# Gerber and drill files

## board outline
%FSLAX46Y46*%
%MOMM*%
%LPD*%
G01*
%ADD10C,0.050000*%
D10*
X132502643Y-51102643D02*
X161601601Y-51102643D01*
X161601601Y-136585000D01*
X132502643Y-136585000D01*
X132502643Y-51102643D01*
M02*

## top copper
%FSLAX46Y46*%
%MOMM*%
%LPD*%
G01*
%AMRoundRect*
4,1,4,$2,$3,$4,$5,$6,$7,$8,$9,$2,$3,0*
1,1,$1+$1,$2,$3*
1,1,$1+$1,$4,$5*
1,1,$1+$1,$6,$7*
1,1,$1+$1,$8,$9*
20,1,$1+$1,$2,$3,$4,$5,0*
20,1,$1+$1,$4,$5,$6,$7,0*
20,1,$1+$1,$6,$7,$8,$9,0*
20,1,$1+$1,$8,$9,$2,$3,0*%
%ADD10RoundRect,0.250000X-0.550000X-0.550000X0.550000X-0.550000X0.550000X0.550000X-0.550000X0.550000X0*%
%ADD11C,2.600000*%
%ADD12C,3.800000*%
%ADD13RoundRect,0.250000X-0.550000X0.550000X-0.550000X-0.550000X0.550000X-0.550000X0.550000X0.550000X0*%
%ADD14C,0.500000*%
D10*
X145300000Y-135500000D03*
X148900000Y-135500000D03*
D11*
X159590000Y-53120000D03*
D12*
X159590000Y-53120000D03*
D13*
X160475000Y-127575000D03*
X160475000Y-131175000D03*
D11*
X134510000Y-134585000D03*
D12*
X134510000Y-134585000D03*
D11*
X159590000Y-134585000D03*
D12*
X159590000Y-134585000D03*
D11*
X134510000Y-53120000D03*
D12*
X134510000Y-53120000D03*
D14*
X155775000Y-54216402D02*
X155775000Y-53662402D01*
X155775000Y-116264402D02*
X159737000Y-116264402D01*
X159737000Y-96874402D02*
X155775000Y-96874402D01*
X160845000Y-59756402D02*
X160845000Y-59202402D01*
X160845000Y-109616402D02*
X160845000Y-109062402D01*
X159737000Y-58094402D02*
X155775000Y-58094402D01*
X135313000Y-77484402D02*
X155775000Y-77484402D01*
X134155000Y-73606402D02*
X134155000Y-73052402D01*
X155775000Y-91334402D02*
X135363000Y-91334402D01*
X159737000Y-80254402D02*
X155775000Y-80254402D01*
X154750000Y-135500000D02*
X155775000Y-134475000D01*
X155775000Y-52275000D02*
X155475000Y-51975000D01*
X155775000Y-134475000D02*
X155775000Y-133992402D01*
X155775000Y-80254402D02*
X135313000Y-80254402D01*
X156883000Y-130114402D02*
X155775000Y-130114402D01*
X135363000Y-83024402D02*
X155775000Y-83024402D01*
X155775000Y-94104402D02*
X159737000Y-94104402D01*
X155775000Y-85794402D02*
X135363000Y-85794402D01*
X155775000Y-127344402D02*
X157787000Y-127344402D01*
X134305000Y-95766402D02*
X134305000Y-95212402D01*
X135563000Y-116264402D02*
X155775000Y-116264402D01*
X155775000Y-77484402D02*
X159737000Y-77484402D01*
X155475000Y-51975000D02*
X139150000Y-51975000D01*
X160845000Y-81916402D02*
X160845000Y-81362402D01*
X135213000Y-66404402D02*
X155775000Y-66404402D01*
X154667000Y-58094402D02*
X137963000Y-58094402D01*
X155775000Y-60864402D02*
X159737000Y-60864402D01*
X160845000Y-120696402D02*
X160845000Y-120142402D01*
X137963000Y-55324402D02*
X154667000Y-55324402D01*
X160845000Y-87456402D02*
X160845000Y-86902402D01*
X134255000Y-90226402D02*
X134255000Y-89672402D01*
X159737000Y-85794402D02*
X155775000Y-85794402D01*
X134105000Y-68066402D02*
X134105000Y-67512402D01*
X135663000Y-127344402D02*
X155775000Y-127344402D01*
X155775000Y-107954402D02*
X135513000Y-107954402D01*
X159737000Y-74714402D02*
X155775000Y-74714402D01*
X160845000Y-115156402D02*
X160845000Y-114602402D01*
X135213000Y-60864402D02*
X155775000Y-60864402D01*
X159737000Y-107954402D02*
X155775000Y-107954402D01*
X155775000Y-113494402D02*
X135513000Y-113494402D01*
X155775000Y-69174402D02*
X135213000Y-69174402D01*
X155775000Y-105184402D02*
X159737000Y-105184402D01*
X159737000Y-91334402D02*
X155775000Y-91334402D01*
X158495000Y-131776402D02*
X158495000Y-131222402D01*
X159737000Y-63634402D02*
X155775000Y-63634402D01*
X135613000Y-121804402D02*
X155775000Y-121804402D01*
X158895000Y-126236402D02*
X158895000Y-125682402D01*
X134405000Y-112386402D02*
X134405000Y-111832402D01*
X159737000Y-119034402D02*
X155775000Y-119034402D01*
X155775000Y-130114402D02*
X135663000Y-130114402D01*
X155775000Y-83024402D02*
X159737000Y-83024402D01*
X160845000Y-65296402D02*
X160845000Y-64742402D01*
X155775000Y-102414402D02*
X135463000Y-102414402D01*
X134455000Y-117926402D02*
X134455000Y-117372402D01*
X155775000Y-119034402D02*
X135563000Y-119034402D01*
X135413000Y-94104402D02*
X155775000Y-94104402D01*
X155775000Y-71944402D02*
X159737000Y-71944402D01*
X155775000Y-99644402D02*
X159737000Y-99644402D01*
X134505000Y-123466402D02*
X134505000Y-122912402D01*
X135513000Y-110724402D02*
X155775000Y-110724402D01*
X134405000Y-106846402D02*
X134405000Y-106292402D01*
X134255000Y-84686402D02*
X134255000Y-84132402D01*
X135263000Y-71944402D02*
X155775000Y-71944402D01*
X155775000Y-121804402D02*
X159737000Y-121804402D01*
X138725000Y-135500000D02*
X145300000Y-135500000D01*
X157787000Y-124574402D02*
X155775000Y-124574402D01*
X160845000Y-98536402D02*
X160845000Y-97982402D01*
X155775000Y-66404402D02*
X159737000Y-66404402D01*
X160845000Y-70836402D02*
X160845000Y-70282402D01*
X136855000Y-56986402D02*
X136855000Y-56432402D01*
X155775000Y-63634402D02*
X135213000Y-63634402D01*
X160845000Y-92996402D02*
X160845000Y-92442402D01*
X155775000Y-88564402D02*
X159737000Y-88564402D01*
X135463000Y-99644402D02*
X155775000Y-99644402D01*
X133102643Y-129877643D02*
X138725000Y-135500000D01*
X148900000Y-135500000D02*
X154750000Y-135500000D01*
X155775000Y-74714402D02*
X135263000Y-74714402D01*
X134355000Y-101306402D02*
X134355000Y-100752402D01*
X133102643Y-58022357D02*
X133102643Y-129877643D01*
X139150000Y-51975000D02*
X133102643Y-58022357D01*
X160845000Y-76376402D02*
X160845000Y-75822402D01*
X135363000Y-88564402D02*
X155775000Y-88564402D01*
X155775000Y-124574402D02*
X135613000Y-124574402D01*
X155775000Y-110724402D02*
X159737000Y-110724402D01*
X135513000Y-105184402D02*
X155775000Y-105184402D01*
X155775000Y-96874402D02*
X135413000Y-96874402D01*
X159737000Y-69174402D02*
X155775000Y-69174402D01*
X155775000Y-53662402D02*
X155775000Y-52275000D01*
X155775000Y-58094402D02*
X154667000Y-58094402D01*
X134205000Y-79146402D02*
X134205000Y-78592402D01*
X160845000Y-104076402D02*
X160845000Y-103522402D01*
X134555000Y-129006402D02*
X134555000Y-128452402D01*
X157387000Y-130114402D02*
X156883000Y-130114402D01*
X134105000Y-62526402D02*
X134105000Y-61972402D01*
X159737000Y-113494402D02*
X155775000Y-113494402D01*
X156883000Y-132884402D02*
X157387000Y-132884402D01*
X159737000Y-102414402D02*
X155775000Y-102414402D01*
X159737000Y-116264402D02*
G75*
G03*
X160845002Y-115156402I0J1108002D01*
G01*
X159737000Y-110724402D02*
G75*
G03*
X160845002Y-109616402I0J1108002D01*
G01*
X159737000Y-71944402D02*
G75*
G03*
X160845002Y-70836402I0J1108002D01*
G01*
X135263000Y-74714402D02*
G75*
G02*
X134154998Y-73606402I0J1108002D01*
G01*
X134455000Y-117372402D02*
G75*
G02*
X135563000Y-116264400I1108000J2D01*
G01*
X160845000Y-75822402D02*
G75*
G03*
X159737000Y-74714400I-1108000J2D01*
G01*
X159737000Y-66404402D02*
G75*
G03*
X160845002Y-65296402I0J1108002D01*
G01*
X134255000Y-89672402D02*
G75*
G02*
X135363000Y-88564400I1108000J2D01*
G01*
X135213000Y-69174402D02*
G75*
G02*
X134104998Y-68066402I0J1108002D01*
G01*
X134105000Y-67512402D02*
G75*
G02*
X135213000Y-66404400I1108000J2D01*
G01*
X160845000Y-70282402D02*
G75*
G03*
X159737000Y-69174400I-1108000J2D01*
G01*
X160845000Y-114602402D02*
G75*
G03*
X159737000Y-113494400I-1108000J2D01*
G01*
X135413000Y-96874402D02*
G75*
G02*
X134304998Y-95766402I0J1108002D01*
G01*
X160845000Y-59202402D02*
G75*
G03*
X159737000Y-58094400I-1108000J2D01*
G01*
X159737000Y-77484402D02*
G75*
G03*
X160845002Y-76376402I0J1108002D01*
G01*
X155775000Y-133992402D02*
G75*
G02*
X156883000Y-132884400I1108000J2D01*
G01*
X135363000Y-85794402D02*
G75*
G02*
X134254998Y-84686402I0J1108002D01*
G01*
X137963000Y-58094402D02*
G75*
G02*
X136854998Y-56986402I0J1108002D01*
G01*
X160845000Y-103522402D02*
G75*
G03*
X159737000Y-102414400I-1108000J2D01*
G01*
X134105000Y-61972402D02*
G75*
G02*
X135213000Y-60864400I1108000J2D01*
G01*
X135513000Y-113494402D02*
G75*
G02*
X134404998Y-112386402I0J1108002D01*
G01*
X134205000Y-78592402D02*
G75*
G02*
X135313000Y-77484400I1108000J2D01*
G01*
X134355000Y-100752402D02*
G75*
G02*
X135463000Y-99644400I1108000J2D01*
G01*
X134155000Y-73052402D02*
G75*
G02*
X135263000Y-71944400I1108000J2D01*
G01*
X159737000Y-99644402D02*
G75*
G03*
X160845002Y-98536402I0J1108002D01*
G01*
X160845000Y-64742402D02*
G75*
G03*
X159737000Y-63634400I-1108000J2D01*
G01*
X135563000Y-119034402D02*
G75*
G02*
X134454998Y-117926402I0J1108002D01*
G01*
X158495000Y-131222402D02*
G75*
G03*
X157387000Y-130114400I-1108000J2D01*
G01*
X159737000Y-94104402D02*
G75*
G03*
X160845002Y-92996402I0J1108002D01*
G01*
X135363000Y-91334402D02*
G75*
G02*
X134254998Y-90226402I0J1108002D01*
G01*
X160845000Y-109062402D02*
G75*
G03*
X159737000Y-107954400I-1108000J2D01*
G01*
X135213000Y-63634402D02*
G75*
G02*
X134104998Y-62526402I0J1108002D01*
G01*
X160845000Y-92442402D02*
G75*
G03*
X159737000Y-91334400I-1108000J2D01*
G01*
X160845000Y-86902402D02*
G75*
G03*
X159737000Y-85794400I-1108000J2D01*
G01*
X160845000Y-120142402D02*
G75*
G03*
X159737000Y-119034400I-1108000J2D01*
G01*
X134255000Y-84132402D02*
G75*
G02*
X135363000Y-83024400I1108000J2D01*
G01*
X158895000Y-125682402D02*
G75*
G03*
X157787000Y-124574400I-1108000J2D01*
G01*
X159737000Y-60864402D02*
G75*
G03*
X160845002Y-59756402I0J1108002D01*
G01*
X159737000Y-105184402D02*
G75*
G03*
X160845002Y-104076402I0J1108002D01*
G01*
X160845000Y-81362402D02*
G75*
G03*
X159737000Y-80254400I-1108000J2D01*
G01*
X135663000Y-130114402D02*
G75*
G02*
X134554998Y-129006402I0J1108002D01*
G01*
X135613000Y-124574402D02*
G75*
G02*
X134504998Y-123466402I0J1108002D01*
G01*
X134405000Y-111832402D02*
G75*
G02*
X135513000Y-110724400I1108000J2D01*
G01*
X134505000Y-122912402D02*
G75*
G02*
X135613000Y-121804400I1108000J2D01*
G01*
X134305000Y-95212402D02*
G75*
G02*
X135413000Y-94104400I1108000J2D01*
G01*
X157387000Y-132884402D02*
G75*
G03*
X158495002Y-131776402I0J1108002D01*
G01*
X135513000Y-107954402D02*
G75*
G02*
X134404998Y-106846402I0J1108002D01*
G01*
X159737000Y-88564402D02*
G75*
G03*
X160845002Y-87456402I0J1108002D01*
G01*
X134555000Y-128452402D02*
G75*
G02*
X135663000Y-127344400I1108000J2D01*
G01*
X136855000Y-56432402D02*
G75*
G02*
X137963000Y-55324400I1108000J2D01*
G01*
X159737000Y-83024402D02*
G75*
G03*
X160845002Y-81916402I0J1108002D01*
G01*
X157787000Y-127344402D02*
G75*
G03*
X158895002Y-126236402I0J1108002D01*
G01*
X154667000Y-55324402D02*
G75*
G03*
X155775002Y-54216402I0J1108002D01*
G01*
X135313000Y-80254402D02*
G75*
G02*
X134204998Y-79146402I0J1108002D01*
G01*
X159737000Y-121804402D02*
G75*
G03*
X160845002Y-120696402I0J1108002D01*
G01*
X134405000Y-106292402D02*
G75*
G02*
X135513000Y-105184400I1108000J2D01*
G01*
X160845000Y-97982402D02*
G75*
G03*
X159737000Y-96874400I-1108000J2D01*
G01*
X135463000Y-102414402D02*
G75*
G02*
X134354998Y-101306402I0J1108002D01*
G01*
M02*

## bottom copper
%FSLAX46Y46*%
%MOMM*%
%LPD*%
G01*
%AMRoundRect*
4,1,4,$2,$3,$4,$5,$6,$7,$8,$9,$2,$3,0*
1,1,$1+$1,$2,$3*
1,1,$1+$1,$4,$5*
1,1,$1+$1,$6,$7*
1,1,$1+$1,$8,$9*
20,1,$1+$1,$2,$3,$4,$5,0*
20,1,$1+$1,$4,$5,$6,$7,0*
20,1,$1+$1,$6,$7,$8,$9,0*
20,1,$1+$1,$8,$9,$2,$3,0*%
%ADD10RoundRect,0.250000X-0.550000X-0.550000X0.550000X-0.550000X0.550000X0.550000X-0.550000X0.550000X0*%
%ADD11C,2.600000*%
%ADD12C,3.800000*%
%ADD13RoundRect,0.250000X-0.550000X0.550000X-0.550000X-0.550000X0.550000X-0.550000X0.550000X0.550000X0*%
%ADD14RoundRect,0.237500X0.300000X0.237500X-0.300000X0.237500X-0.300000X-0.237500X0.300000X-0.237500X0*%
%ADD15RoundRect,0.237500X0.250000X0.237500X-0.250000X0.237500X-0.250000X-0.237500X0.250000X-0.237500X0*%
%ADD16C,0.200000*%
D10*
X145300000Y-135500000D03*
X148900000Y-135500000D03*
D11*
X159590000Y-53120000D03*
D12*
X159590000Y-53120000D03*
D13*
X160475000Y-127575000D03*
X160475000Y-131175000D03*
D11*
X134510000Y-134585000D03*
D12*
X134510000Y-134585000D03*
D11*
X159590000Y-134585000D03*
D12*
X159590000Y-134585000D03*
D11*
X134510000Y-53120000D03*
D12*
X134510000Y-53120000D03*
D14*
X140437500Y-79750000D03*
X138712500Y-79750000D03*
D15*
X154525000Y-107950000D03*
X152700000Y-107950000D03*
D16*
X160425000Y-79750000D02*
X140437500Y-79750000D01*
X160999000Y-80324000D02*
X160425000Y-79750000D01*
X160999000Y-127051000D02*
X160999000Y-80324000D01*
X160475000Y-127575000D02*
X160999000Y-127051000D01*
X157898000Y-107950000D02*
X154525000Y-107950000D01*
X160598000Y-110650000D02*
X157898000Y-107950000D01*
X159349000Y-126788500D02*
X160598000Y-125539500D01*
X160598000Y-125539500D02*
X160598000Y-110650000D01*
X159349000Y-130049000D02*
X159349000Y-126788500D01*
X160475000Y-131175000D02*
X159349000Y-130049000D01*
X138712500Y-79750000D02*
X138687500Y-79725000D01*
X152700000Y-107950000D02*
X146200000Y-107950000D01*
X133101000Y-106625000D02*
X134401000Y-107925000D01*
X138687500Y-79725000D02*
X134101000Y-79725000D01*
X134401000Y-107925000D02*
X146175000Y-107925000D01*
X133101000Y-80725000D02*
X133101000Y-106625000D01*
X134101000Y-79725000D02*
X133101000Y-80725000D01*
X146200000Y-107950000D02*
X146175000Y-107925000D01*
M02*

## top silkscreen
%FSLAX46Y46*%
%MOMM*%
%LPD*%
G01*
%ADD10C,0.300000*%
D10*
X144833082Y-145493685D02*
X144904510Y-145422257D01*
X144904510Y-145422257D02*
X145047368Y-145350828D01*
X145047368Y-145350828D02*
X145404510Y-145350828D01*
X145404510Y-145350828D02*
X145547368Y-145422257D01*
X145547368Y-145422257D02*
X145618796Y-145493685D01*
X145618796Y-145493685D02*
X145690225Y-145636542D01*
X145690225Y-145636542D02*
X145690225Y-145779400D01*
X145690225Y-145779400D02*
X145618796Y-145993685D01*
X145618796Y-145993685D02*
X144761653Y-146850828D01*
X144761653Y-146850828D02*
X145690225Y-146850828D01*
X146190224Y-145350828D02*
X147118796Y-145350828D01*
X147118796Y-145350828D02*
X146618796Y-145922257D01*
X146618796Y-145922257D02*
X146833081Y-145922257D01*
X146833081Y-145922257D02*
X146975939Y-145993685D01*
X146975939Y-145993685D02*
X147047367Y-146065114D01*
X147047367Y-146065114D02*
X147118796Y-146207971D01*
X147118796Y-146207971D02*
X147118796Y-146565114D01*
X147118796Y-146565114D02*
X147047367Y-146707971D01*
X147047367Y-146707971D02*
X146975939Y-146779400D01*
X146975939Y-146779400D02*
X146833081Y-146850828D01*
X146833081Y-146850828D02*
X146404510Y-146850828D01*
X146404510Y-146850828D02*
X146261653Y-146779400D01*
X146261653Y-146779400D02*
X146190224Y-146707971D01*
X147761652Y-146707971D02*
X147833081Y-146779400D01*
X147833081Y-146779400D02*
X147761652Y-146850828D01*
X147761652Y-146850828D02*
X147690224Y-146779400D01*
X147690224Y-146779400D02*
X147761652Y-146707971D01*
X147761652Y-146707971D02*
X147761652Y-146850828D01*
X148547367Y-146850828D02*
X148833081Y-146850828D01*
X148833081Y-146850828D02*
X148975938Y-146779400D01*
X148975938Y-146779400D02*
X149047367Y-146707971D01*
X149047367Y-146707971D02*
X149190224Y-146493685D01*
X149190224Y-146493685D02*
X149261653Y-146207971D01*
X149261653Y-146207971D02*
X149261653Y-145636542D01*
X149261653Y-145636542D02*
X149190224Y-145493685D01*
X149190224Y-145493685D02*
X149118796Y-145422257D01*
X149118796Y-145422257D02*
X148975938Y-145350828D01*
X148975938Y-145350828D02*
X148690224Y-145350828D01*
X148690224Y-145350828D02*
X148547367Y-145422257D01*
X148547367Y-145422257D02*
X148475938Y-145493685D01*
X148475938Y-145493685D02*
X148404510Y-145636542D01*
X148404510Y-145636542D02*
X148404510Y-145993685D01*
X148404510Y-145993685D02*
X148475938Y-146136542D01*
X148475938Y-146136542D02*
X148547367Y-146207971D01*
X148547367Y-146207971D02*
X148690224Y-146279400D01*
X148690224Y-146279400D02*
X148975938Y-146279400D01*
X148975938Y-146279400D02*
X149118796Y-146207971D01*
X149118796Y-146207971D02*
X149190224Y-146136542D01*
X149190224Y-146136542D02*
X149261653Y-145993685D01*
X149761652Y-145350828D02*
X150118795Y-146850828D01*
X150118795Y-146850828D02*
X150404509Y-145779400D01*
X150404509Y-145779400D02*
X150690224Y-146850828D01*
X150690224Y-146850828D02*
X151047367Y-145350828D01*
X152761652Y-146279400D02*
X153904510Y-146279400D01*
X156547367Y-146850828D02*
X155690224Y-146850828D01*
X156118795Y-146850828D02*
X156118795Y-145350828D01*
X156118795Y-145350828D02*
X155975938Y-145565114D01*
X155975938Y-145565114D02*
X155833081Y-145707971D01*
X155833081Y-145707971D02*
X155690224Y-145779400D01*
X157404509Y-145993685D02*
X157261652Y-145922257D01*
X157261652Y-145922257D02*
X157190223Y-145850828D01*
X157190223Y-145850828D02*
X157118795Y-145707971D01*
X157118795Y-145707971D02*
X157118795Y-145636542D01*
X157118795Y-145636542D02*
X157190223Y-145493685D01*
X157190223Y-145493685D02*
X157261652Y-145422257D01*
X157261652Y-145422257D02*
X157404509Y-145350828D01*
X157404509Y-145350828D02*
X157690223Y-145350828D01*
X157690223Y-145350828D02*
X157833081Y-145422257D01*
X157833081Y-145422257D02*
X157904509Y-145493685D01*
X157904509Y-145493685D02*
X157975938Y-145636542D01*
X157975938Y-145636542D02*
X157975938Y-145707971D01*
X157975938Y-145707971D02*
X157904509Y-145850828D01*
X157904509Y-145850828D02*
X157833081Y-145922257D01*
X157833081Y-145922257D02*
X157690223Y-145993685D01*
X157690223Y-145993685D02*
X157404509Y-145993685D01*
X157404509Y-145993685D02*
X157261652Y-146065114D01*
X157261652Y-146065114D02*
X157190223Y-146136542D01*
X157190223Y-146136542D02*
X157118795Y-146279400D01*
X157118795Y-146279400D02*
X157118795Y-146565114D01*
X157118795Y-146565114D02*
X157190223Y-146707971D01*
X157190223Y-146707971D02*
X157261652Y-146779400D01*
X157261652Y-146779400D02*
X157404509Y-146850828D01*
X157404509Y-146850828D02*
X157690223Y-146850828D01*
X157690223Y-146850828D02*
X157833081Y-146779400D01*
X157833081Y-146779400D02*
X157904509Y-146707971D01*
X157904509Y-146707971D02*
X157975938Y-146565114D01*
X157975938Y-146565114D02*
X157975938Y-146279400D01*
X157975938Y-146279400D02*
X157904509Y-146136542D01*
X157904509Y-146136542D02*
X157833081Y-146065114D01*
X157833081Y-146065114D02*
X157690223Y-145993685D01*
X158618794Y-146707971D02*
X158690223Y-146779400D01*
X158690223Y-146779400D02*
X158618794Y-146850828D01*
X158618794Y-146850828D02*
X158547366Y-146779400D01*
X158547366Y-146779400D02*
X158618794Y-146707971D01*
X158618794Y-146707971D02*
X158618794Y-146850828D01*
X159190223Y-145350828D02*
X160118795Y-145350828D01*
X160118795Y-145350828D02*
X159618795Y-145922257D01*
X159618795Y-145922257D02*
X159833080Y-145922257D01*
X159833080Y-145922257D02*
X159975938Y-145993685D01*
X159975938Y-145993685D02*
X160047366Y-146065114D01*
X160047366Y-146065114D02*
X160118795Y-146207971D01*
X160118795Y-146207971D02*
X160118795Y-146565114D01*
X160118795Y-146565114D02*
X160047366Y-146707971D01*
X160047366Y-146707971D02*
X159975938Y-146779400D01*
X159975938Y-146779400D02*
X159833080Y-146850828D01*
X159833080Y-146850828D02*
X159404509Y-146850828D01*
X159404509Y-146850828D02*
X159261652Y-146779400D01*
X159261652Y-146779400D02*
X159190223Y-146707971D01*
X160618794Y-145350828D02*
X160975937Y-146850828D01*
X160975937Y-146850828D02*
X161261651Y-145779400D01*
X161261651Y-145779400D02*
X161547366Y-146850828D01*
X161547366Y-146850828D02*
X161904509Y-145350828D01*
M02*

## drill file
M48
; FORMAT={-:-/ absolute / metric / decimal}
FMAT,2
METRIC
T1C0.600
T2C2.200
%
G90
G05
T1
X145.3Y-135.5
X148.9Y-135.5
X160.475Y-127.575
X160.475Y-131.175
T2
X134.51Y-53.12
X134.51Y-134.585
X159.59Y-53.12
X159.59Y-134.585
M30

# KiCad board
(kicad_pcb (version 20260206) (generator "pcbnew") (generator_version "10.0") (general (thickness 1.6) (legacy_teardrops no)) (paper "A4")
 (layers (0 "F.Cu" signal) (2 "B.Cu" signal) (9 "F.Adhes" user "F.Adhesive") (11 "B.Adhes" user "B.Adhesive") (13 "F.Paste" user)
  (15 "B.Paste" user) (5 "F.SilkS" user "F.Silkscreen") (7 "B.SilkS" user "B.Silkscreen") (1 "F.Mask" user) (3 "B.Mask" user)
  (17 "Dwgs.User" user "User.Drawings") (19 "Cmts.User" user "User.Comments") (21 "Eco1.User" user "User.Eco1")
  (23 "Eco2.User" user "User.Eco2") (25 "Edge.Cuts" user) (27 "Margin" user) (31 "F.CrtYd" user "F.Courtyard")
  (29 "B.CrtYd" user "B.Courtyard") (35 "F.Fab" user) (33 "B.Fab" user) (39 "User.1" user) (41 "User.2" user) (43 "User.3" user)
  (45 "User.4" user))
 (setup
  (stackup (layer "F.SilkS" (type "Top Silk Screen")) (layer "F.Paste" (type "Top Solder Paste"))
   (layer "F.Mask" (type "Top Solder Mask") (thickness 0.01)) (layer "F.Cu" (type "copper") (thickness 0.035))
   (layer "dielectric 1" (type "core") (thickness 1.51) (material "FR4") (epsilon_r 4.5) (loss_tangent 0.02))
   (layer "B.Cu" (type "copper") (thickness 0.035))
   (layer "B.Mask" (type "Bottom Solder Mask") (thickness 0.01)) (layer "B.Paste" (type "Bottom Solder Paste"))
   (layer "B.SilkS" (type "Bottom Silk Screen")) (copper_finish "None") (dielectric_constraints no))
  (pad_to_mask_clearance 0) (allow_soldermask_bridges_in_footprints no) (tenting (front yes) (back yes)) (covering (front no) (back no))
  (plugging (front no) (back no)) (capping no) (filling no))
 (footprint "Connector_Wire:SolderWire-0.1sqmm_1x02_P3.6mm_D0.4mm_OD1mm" (layer "F.Cu") (at 145.3 135.5)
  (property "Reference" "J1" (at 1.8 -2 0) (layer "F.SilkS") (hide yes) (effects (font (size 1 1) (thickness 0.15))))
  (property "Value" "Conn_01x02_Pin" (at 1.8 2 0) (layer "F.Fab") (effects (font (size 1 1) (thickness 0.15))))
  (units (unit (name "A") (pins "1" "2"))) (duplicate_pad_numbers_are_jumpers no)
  (pad "1" thru_hole roundrect (at 0 0) (size 1.6 1.6) (drill 0.6) (layers "*.Cu" "*.Mask") (remove_unused_layers no)
   (roundrect_rratio 0.15625) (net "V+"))
  (pad "2" thru_hole roundrect (at 3.6 0) (size 1.6 1.6) (drill 0.6) (layers "*.Cu" "*.Mask") (remove_unused_layers no)
   (roundrect_rratio 0.15625) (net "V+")))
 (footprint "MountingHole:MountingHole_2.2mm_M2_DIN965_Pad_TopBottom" (layer "F.Cu") (at 159.59 53.12)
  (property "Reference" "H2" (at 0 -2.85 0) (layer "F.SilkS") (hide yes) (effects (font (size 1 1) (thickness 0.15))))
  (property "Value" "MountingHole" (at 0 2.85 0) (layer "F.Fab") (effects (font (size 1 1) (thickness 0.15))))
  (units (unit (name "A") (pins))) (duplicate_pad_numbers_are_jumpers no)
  (pad "1" thru_hole circle (at 0 0) (size 2.6 2.6) (drill 2.2) (layers "*.Cu" "*.Mask") (remove_unused_layers no) (zone_connect 2))
  (pad "1" connect circle (at 0 0) (size 3.8 3.8) (layers "F.Cu" "F.Mask") (zone_connect 2))
  (pad "1" connect circle (at 0 0) (size 3.8 3.8) (layers "B.Cu" "B.Mask") (zone_connect 2)))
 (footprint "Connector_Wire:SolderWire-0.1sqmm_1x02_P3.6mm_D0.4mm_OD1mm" (layer "F.Cu") (at 160.475 127.575 -90)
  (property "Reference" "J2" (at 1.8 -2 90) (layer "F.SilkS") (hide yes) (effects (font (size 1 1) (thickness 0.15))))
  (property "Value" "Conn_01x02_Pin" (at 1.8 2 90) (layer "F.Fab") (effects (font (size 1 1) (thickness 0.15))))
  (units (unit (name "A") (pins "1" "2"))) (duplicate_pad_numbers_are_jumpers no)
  (pad "1" thru_hole roundrect (at 0 0 270) (size 1.6 1.6) (drill 0.6) (layers "*.Cu" "*.Mask") (remove_unused_layers no)
   (roundrect_rratio 0.15625) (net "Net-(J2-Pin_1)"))
  (pad "2" thru_hole roundrect (at 3.6 0 270) (size 1.6 1.6) (drill 0.6) (layers "*.Cu" "*.Mask") (remove_unused_layers no)
   (roundrect_rratio 0.15625) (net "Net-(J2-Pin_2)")))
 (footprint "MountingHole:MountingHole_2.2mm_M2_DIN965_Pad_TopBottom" (layer "F.Cu") (at 134.51 134.585)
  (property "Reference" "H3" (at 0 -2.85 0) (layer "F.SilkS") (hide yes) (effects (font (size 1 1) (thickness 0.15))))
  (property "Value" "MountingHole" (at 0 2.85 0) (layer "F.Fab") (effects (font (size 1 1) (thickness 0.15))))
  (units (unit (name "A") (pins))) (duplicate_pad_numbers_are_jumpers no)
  (pad "1" thru_hole circle (at 0 0) (size 2.6 2.6) (drill 2.2) (layers "*.Cu" "*.Mask") (remove_unused_layers no) (zone_connect 2))
  (pad "1" connect circle (at 0 0) (size 3.8 3.8) (layers "F.Cu" "F.Mask") (zone_connect 2))
  (pad "1" connect circle (at 0 0) (size 3.8 3.8) (layers "B.Cu" "B.Mask") (zone_connect 2)))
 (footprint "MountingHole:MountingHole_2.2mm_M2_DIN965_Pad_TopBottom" (layer "F.Cu") (at 159.59 134.585)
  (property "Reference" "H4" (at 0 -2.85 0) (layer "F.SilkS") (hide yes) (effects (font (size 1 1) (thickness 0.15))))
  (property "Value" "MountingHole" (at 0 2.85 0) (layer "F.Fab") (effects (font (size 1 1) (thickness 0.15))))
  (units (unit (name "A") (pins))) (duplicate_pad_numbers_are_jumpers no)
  (pad "1" thru_hole circle (at 0 0) (size 2.6 2.6) (drill 2.2) (layers "*.Cu" "*.Mask") (remove_unused_layers no) (zone_connect 2))
  (pad "1" connect circle (at 0 0) (size 3.8 3.8) (layers "F.Cu" "F.Mask") (zone_connect 2))
  (pad "1" connect circle (at 0 0) (size 3.8 3.8) (layers "B.Cu" "B.Mask") (zone_connect 2)))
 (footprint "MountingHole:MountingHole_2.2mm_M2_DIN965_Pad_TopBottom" (layer "F.Cu") (at 134.51 53.12)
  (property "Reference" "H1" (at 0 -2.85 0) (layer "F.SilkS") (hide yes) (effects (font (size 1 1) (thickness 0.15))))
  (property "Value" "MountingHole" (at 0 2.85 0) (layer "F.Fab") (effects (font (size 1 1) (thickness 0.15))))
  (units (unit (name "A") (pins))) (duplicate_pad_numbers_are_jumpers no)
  (pad "1" thru_hole circle (at 0 0) (size 2.6 2.6) (drill 2.2) (layers "*.Cu" "*.Mask") (remove_unused_layers no) (zone_connect 2))
  (pad "1" connect circle (at 0 0) (size 3.8 3.8) (layers "F.Cu" "F.Mask") (zone_connect 2))
  (pad "1" connect circle (at 0 0) (size 3.8 3.8) (layers "B.Cu" "B.Mask") (zone_connect 2)))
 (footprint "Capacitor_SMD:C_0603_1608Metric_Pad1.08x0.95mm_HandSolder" (layer "B.Cu") (at 139.575 79.75 180)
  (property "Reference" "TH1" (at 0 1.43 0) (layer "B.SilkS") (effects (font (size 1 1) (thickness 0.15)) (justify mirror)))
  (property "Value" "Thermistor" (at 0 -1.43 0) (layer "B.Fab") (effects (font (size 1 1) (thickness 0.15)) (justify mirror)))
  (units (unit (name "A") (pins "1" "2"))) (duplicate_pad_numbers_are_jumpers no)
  (pad "1" smd roundrect (at -0.8625 0 180) (size 1.075 0.95) (layers "B.Cu" "B.Mask" "B.Paste") (roundrect_rratio 0.25)
   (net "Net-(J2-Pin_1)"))
  (pad "2" smd roundrect (at 0.8625 0 180) (size 1.075 0.95) (layers "B.Cu" "B.Mask" "B.Paste") (roundrect_rratio 0.25)
   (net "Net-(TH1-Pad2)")))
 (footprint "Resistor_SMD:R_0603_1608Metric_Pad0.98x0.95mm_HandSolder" (layer "B.Cu") (at 153.6125 107.95 180)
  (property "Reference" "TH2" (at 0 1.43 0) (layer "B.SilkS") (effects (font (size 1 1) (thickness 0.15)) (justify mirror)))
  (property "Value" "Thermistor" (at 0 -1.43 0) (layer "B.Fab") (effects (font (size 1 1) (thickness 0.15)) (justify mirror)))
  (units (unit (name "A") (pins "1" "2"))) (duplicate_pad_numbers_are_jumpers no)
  (pad "1" smd roundrect (at -0.9125 0 180) (size 0.975 0.95) (layers "B.Cu" "B.Mask" "B.Paste") (roundrect_rratio 0.25)
   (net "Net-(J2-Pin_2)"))
  (pad "2" smd roundrect (at 0.9125 0 180) (size 0.975 0.95) (layers "B.Cu" "B.Mask" "B.Paste") (roundrect_rratio 0.25)
   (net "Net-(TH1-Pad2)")))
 (gr_rect (start 132.502643 51.102643) (end 161.601601 136.585) (stroke (width 0.05) (type default)) (fill no) (layer "Edge.Cuts"))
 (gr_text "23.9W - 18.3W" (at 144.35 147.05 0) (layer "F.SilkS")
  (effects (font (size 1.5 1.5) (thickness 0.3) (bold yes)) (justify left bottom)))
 (segment (start 155.775 54.216402) (end 155.775 53.662402) (width 0.5) (layer "F.Cu") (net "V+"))
 (segment (start 155.775 116.264402) (end 159.737 116.264402) (width 0.5) (layer "F.Cu") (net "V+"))
 (segment (start 159.737 96.874402) (end 155.775 96.874402) (width 0.5) (layer "F.Cu") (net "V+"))
 (segment (start 160.845 59.756402) (end 160.845 59.202402) (width 0.5) (layer "F.Cu") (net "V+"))
 (segment (start 160.845 109.616402) (end 160.845 109.062402) (width 0.5) (layer "F.Cu") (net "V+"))
 (segment (start 159.737 58.094402) (end 155.775 58.094402) (width 0.5) (layer "F.Cu") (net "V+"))
 (segment (start 135.313 77.484402) (end 155.775 77.484402) (width 0.5) (layer "F.Cu") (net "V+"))
 (segment (start 134.155 73.606402) (end 134.155 73.052402) (width 0.5) (layer "F.Cu") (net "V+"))
 (segment (start 155.775 91.334402) (end 135.363 91.334402) (width 0.5) (layer "F.Cu") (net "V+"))
 (segment (start 159.737 80.254402) (end 155.775 80.254402) (width 0.5) (layer "F.Cu") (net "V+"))
 (segment (start 154.75 135.5) (end 155.775 134.475) (width 0.5) (layer "F.Cu") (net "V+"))
 (segment (start 155.775 52.275) (end 155.475 51.975) (width 0.5) (layer "F.Cu") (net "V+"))
 (segment (start 155.775 134.475) (end 155.775 133.992402) (width 0.5) (layer "F.Cu") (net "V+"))
 (segment (start 155.775 80.254402) (end 135.313 80.254402) (width 0.5) (layer "F.Cu") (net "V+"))
 (segment (start 156.883 130.114402) (end 155.775 130.114402) (width 0.5) (layer "F.Cu") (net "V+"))
 (segment (start 135.363 83.024402) (end 155.775 83.024402) (width 0.5) (layer "F.Cu") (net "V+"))
 (segment (start 155.775 94.104402) (end 159.737 94.104402) (width 0.5) (layer "F.Cu") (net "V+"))
 (segment (start 155.775 85.794402) (end 135.363 85.794402) (width 0.5) (layer "F.Cu") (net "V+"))
 (segment (start 155.775 127.344402) (end 157.787 127.344402) (width 0.5) (layer "F.Cu") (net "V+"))
 (segment (start 134.305 95.766402) (end 134.305 95.212402) (width 0.5) (layer "F.Cu") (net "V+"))
 (segment (start 135.563 116.264402) (end 155.775 116.264402) (width 0.5) (layer "F.Cu") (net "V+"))
 (segment (start 155.775 77.484402) (end 159.737 77.484402) (width 0.5) (layer "F.Cu") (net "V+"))
 (segment (start 155.475 51.975) (end 139.15 51.975) (width 0.5) (layer "F.Cu") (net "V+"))
 (segment (start 160.845 81.916402) (end 160.845 81.362402) (width 0.5) (layer "F.Cu") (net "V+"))
 (segment (start 135.213 66.404402) (end 155.775 66.404402) (width 0.5) (layer "F.Cu") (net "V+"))
 (segment (start 154.667 58.094402) (end 137.963 58.094402) (width 0.5) (layer "F.Cu") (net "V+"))
 (segment (start 155.775 60.864402) (end 159.737 60.864402) (width 0.5) (layer "F.Cu") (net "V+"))
 (segment (start 160.845 120.696402) (end 160.845 120.142402) (width 0.5) (layer "F.Cu") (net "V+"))
 (segment (start 137.963 55.324402) (end 154.667 55.324402) (width 0.5) (layer "F.Cu") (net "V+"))
 (segment (start 160.845 87.456402) (end 160.845 86.902402) (width 0.5) (layer "F.Cu") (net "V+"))
 (segment (start 134.255 90.226402) (end 134.255 89.672402) (width 0.5) (layer "F.Cu") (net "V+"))
 (segment (start 159.737 85.794402) (end 155.775 85.794402) (width 0.5) (layer "F.Cu") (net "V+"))
 (segment (start 134.105 68.066402) (end 134.105 67.512402) (width 0.5) (layer "F.Cu") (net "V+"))
 (segment (start 135.663 127.344402) (end 155.775 127.344402) (width 0.5) (layer "F.Cu") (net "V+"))
 (segment (start 155.775 107.954402) (end 135.513 107.954402) (width 0.5) (layer "F.Cu") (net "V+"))
 (segment (start 159.737 74.714402) (end 155.775 74.714402) (width 0.5) (layer "F.Cu") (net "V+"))
 (segment (start 160.845 115.156402) (end 160.845 114.602402) (width 0.5) (layer "F.Cu") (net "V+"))
 (segment (start 135.213 60.864402) (end 155.775 60.864402) (width 0.5) (layer "F.Cu") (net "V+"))
 (segment (start 159.737 107.954402) (end 155.775 107.954402) (width 0.5) (layer "F.Cu") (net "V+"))
 (segment (start 155.775 113.494402) (end 135.513 113.494402) (width 0.5) (layer "F.Cu") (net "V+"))
 (segment (start 155.775 69.174402) (end 135.213 69.174402) (width 0.5) (layer "F.Cu") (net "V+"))
 (segment (start 155.775 105.184402) (end 159.737 105.184402) (width 0.5) (layer "F.Cu") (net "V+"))
 (segment (start 159.737 91.334402) (end 155.775 91.334402) (width 0.5) (layer "F.Cu") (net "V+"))
 (segment (start 158.495 131.776402) (end 158.495 131.222402) (width 0.5) (layer "F.Cu") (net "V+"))
 (segment (start 159.737 63.634402) (end 155.775 63.634402) (width 0.5) (layer "F.Cu") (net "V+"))
 (segment (start 135.613 121.804402) (end 155.775 121.804402) (width 0.5) (layer "F.Cu") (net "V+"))
 (segment (start 158.895 126.236402) (end 158.895 125.682402) (width 0.5) (layer "F.Cu") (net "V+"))
 (segment (start 134.405 112.386402) (end 134.405 111.832402) (width 0.5) (layer "F.Cu") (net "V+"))
 (segment (start 159.737 119.034402) (end 155.775 119.034402) (width 0.5) (layer "F.Cu") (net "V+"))
 (segment (start 155.775 130.114402) (end 135.663 130.114402) (width 0.5) (layer "F.Cu") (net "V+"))
 (segment (start 155.775 83.024402) (end 159.737 83.024402) (width 0.5) (layer "F.Cu") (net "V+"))
 (segment (start 160.845 65.296402) (end 160.845 64.742402) (width 0.5) (layer "F.Cu") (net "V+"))
 (segment (start 155.775 102.414402) (end 135.463 102.414402) (width 0.5) (layer "F.Cu") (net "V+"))
 (segment (start 134.455 117.926402) (end 134.455 117.372402) (width 0.5) (layer "F.Cu") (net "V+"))
 (segment (start 155.775 119.034402) (end 135.563 119.034402) (width 0.5) (layer "F.Cu") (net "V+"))
 (segment (start 135.413 94.104402) (end 155.775 94.104402) (width 0.5) (layer "F.Cu") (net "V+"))
 (segment (start 155.775 71.944402) (end 159.737 71.944402) (width 0.5) (layer "F.Cu") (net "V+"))
 (segment (start 155.775 99.644402) (end 159.737 99.644402) (width 0.5) (layer "F.Cu") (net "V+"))
 (segment (start 134.505 123.466402) (end 134.505 122.912402) (width 0.5) (layer "F.Cu") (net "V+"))
 (segment (start 135.513 110.724402) (end 155.775 110.724402) (width 0.5) (layer "F.Cu") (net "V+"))
 (segment (start 134.405 106.846402) (end 134.405 106.292402) (width 0.5) (layer "F.Cu") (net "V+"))
 (segment (start 134.255 84.686402) (end 134.255 84.132402) (width 0.5) (layer "F.Cu") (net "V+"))
 (segment (start 135.263 71.944402) (end 155.775 71.944402) (width 0.5) (layer "F.Cu") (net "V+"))
 (segment (start 155.775 121.804402) (end 159.737 121.804402) (width 0.5) (layer "F.Cu") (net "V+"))
 (segment (start 138.725 135.5) (end 145.3 135.5) (width 0.5) (layer "F.Cu") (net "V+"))
 (segment (start 157.787 124.574402) (end 155.775 124.574402) (width 0.5) (layer "F.Cu") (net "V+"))
 (segment (start 160.845 98.536402) (end 160.845 97.982402) (width 0.5) (layer "F.Cu") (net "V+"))
 (segment (start 155.775 66.404402) (end 159.737 66.404402) (width 0.5) (layer "F.Cu") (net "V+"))
 (segment (start 160.845 70.836402) (end 160.845 70.282402) (width 0.5) (layer "F.Cu") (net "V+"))
 (segment (start 136.855 56.986402) (end 136.855 56.432402) (width 0.5) (layer "F.Cu") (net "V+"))
 (segment (start 155.775 63.634402) (end 135.213 63.634402) (width 0.5) (layer "F.Cu") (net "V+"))
 (segment (start 160.845 92.996402) (end 160.845 92.442402) (width 0.5) (layer "F.Cu") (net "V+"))
 (segment (start 155.775 88.564402) (end 159.737 88.564402) (width 0.5) (layer "F.Cu") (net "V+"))
 (segment (start 135.463 99.644402) (end 155.775 99.644402) (width 0.5) (layer "F.Cu") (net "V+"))
 (segment (start 133.102643 129.877643) (end 138.725 135.5) (width 0.5) (layer "F.Cu") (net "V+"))
 (segment (start 148.9 135.5) (end 154.75 135.5) (width 0.5) (layer "F.Cu") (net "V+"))
 (segment (start 155.775 74.714402) (end 135.263 74.714402) (width 0.5) (layer "F.Cu") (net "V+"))
 (segment (start 134.355 101.306402) (end 134.355 100.752402) (width 0.5) (layer "F.Cu") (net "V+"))
 (segment (start 133.102643 58.022357) (end 133.102643 129.877643) (width 0.5) (layer "F.Cu") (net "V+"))
 (segment (start 139.15 51.975) (end 133.102643 58.022357) (width 0.5) (layer "F.Cu") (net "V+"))
 (segment (start 160.845 76.376402) (end 160.845 75.822402) (width 0.5) (layer "F.Cu") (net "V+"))
 (segment (start 135.363 88.564402) (end 155.775 88.564402) (width 0.5) (layer "F.Cu") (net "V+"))
 (segment (start 155.775 124.574402) (end 135.613 124.574402) (width 0.5) (layer "F.Cu") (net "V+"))
 (segment (start 155.775 110.724402) (end 159.737 110.724402) (width 0.5) (layer "F.Cu") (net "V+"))
 (segment (start 135.513 105.184402) (end 155.775 105.184402) (width 0.5) (layer "F.Cu") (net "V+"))
 (segment (start 155.775 96.874402) (end 135.413 96.874402) (width 0.5) (layer "F.Cu") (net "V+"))
 (segment (start 159.737 69.174402) (end 155.775 69.174402) (width 0.5) (layer "F.Cu") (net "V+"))
 (segment (start 155.775 53.662402) (end 155.775 52.275) (width 0.5) (layer "F.Cu") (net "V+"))
 (segment (start 155.775 58.094402) (end 154.667 58.094402) (width 0.5) (layer "F.Cu") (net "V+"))
 (segment (start 134.205 79.146402) (end 134.205 78.592402) (width 0.5) (layer "F.Cu") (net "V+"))
 (segment (start 160.845 104.076402) (end 160.845 103.522402) (width 0.5) (layer "F.Cu") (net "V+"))
 (segment (start 134.555 129.006402) (end 134.555 128.452402) (width 0.5) (layer "F.Cu") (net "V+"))
 (segment (start 157.387 130.114402) (end 156.883 130.114402) (width 0.5) (layer "F.Cu") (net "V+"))
 (segment (start 134.105 62.526402) (end 134.105 61.972402) (width 0.5) (layer "F.Cu") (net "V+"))
 (segment (start 159.737 113.494402) (end 155.775 113.494402) (width 0.5) (layer "F.Cu") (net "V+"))
 (segment (start 156.883 132.884402) (end 157.387 132.884402) (width 0.5) (layer "F.Cu") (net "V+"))
 (segment (start 159.737 102.414402) (end 155.775 102.414402) (width 0.5) (layer "F.Cu") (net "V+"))
 (arc (start 159.737 116.264402) (mid 160.520474 115.939876) (end 160.845 115.156402) (width 0.5) (layer "F.Cu") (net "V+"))
 (arc (start 159.737 110.724402) (mid 160.520474 110.399876) (end 160.845 109.616402) (width 0.5) (layer "F.Cu") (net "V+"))
 (arc (start 159.737 71.944402) (mid 160.520474 71.619876) (end 160.845 70.836402) (width 0.5) (layer "F.Cu") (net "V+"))
 (arc (start 135.263 74.714402) (mid 134.479526 74.389876) (end 134.155 73.606402) (width 0.5) (layer "F.Cu") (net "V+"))
 (arc (start 134.455 117.372402) (mid 134.779526 116.588928) (end 135.563 116.264402) (width 0.5) (layer "F.Cu") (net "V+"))
 (arc (start 160.845 75.822402) (mid 160.520474 75.038928) (end 159.737 74.714402) (width 0.5) (layer "F.Cu") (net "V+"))
 (arc (start 159.737 66.404402) (mid 160.520474 66.079876) (end 160.845 65.296402) (width 0.5) (layer "F.Cu") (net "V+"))
 (arc (start 134.255 89.672402) (mid 134.579526 88.888928) (end 135.363 88.564402) (width 0.5) (layer "F.Cu") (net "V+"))
 (arc (start 135.213 69.174402) (mid 134.429526 68.849876) (end 134.105 68.066402) (width 0.5) (layer "F.Cu") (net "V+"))
 (arc (start 134.105 67.512402) (mid 134.429526 66.728928) (end 135.213 66.404402) (width 0.5) (layer "F.Cu") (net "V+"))
 (arc (start 160.845 70.282402) (mid 160.520474 69.498928) (end 159.737 69.174402) (width 0.5) (layer "F.Cu") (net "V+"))
 (arc (start 160.845 114.602402) (mid 160.520474 113.818928) (end 159.737 113.494402) (width 0.5) (layer "F.Cu") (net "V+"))
 (arc (start 135.413 96.874402) (mid 134.629526 96.549876) (end 134.305 95.766402) (width 0.5) (layer "F.Cu") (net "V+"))
 (arc (start 160.845 59.202402) (mid 160.520474 58.418928) (end 159.737 58.094402) (width 0.5) (layer "F.Cu") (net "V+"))
 (arc (start 159.737 77.484402) (mid 160.520474 77.159876) (end 160.845 76.376402) (width 0.5) (layer "F.Cu") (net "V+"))
 (arc (start 155.775 133.992402) (mid 156.099526 133.208928) (end 156.883 132.884402) (width 0.5) (layer "F.Cu") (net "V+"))
 (arc (start 135.363 85.794402) (mid 134.579526 85.469876) (end 134.255 84.686402) (width 0.5) (layer "F.Cu") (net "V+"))
 (arc (start 137.963 58.094402) (mid 137.179526 57.769876) (end 136.855 56.986402) (width 0.5) (layer "F.Cu") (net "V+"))
 (arc (start 160.845 103.522402) (mid 160.520474 102.738928) (end 159.737 102.414402) (width 0.5) (layer "F.Cu") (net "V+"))
 (arc (start 134.105 61.972402) (mid 134.429526 61.188928) (end 135.213 60.864402) (width 0.5) (layer "F.Cu") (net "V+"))
 (arc (start 135.513 113.494402) (mid 134.729526 113.169876) (end 134.405 112.386402) (width 0.5) (layer "F.Cu") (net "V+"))
 (arc (start 134.205 78.592402) (mid 134.529526 77.808928) (end 135.313 77.484402) (width 0.5) (layer "F.Cu") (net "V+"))
 (arc (start 134.355 100.752402) (mid 134.679526 99.968928) (end 135.463 99.644402) (width 0.5) (layer "F.Cu") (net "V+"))
 (arc (start 134.155 73.052402) (mid 134.479526 72.268928) (end 135.263 71.944402) (width 0.5) (layer "F.Cu") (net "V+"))
 (arc (start 159.737 99.644402) (mid 160.520474 99.319876) (end 160.845 98.536402) (width 0.5) (layer "F.Cu") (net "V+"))
 (arc (start 160.845 64.742402) (mid 160.520474 63.958928) (end 159.737 63.634402) (width 0.5) (layer "F.Cu") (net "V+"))
 (arc (start 135.563 119.034402) (mid 134.779526 118.709876) (end 134.455 117.926402) (width 0.5) (layer "F.Cu") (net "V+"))
 (arc (start 158.495 131.222402) (mid 158.170474 130.438928) (end 157.387 130.114402) (width 0.5) (layer "F.Cu") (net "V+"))
 (arc (start 159.737 94.104402) (mid 160.520474 93.779876) (end 160.845 92.996402) (width 0.5) (layer "F.Cu") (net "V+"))
 (arc (start 135.363 91.334402) (mid 134.579526 91.009876) (end 134.255 90.226402) (width 0.5) (layer "F.Cu") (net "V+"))
 (arc (start 160.845 109.062402) (mid 160.520474 108.278928) (end 159.737 107.954402) (width 0.5) (layer "F.Cu") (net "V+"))
 (arc (start 135.213 63.634402) (mid 134.429526 63.309876) (end 134.105 62.526402) (width 0.5) (layer "F.Cu") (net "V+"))
 (arc (start 160.845 92.442402) (mid 160.520474 91.658928) (end 159.737 91.334402) (width 0.5) (layer "F.Cu") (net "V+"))
 (arc (start 160.845 86.902402) (mid 160.520474 86.118928) (end 159.737 85.794402) (width 0.5) (layer "F.Cu") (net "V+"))
 (arc (start 160.845 120.142402) (mid 160.520474 119.358928) (end 159.737 119.034402) (width 0.5) (layer "F.Cu") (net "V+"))
 (arc (start 134.255 84.132402) (mid 134.579526 83.348928) (end 135.363 83.024402) (width 0.5) (layer "F.Cu") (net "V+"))
 (arc (start 158.895 125.682402) (mid 158.570474 124.898928) (end 157.787 124.574402) (width 0.5) (layer "F.Cu") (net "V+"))
 (arc (start 159.737 60.864402) (mid 160.520474 60.539876) (end 160.845 59.756402) (width 0.5) (layer "F.Cu") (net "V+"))
 (arc (start 159.737 105.184402) (mid 160.520474 104.859876) (end 160.845 104.076402) (width 0.5) (layer "F.Cu") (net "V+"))
 (arc (start 160.845 81.362402) (mid 160.520474 80.578928) (end 159.737 80.254402) (width 0.5) (layer "F.Cu") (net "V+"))
 (arc (start 135.663 130.114402) (mid 134.879526 129.789876) (end 134.555 129.006402) (width 0.5) (layer "F.Cu") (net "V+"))
 (arc (start 135.613 124.574402) (mid 134.829526 124.249876) (end 134.505 123.466402) (width 0.5) (layer "F.Cu") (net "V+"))
 (arc (start 134.405 111.832402) (mid 134.729526 111.048928) (end 135.513 110.724402) (width 0.5) (layer "F.Cu") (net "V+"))
 (arc (start 134.505 122.912402) (mid 134.829526 122.128928) (end 135.613 121.804402) (width 0.5) (layer "F.Cu") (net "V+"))
 (arc (start 134.305 95.212402) (mid 134.629526 94.428928) (end 135.413 94.104402) (width 0.5) (layer "F.Cu") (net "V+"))
 (arc (start 157.387 132.884402) (mid 158.170474 132.559876) (end 158.495 131.776402) (width 0.5) (layer "F.Cu") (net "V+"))
 (arc (start 135.513 107.954402) (mid 134.729526 107.629876) (end 134.405 106.846402) (width 0.5) (layer "F.Cu") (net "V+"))
 (arc (start 159.737 88.564402) (mid 160.520474 88.239876) (end 160.845 87.456402) (width 0.5) (layer "F.Cu") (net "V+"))
 (arc (start 134.555 128.452402) (mid 134.879526 127.668928) (end 135.663 127.344402) (width 0.5) (layer "F.Cu") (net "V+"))
 (arc (start 136.855 56.432402) (mid 137.179526 55.648928) (end 137.963 55.324402) (width 0.5) (layer "F.Cu") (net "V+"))
 (arc (start 159.737 83.024402) (mid 160.520474 82.699876) (end 160.845 81.916402) (width 0.5) (layer "F.Cu") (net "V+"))
 (arc (start 157.787 127.344402) (mid 158.570474 127.019876) (end 158.895 126.236402) (width 0.5) (layer "F.Cu") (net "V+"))
 (arc (start 154.667 55.324402) (mid 155.450474 54.999876) (end 155.775 54.216402) (width 0.5) (layer "F.Cu") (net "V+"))
 (arc (start 135.313 80.254402) (mid 134.529526 79.929876) (end 134.205 79.146402) (width 0.5) (layer "F.Cu") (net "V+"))
 (arc (start 159.737 121.804402) (mid 160.520474 121.479876) (end 160.845 120.696402) (width 0.5) (layer "F.Cu") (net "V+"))
 (arc (start 134.405 106.292402) (mid 134.729526 105.508928) (end 135.513 105.184402) (width 0.5) (layer "F.Cu") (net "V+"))
 (arc (start 160.845 97.982402) (mid 160.520474 97.198928) (end 159.737 96.874402) (width 0.5) (layer "F.Cu") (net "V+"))
 (arc (start 135.463 102.414402) (mid 134.679526 102.089876) (end 134.355 101.306402) (width 0.5) (layer "F.Cu") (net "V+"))
 (segment (start 160.425 79.75) (end 140.4375 79.75) (width 0.2) (layer "B.Cu") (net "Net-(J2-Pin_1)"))
 (segment (start 160.999 80.324) (end 160.425 79.75) (width 0.2) (layer "B.Cu") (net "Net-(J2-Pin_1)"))
 (segment (start 160.999 127.051) (end 160.999 80.324) (width 0.2) (layer "B.Cu") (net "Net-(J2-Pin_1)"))
 (segment (start 160.475 127.575) (end 160.999 127.051) (width 0.2) (layer "B.Cu") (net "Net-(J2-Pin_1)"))
 (segment (start 157.898 107.95) (end 154.525 107.95) (width 0.2) (layer "B.Cu") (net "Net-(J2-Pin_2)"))
 (segment (start 160.598 110.65) (end 157.898 107.95) (width 0.2) (layer "B.Cu") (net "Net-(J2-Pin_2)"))
 (segment (start 159.349 126.7885) (end 160.598 125.5395) (width 0.2) (layer "B.Cu") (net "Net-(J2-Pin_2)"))
 (segment (start 160.598 125.5395) (end 160.598 110.65) (width 0.2) (layer "B.Cu") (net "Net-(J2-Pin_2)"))
 (segment (start 159.349 130.049) (end 159.349 126.7885) (width 0.2) (layer "B.Cu") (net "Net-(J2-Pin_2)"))
 (segment (start 160.475 131.175) (end 159.349 130.049) (width 0.2) (layer "B.Cu") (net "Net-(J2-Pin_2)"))
 (segment (start 138.7125 79.75) (end 138.6875 79.725) (width 0.2) (layer "B.Cu") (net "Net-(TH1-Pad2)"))
 (segment (start 152.7 107.95) (end 146.2 107.95) (width 0.2) (layer "B.Cu") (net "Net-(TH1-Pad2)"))
 (segment (start 133.101 106.625) (end 134.401 107.925) (width 0.2) (layer "B.Cu") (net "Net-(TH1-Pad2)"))
 (segment (start 138.6875 79.725) (end 134.101 79.725) (width 0.2) (layer "B.Cu") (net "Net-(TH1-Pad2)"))
 (segment (start 134.401 107.925) (end 146.175 107.925) (width 0.2) (layer "B.Cu") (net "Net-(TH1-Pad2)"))
 (segment (start 133.101 80.725) (end 133.101 106.625) (width 0.2) (layer "B.Cu") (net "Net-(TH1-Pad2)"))
 (segment (start 134.101 79.725) (end 133.101 80.725) (width 0.2) (layer "B.Cu") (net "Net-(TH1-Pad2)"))
 (segment (start 146.2 107.95) (end 146.175 107.925) (width 0.2) (layer "B.Cu") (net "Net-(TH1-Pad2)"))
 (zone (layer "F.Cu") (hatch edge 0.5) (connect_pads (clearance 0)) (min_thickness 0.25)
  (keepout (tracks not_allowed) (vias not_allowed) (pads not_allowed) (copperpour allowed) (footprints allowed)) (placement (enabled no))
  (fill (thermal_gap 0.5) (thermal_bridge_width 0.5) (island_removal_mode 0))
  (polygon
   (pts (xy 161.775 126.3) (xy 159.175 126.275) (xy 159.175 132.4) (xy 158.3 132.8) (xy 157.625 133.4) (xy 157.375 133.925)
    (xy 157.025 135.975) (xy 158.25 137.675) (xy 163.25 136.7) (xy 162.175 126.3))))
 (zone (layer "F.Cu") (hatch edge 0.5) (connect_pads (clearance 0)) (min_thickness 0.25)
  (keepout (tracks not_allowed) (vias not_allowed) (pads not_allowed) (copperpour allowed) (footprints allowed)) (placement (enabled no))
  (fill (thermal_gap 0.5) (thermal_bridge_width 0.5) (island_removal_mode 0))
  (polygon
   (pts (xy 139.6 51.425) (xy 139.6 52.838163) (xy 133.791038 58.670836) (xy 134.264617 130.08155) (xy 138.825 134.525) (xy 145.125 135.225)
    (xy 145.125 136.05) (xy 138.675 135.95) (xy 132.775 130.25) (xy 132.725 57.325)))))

